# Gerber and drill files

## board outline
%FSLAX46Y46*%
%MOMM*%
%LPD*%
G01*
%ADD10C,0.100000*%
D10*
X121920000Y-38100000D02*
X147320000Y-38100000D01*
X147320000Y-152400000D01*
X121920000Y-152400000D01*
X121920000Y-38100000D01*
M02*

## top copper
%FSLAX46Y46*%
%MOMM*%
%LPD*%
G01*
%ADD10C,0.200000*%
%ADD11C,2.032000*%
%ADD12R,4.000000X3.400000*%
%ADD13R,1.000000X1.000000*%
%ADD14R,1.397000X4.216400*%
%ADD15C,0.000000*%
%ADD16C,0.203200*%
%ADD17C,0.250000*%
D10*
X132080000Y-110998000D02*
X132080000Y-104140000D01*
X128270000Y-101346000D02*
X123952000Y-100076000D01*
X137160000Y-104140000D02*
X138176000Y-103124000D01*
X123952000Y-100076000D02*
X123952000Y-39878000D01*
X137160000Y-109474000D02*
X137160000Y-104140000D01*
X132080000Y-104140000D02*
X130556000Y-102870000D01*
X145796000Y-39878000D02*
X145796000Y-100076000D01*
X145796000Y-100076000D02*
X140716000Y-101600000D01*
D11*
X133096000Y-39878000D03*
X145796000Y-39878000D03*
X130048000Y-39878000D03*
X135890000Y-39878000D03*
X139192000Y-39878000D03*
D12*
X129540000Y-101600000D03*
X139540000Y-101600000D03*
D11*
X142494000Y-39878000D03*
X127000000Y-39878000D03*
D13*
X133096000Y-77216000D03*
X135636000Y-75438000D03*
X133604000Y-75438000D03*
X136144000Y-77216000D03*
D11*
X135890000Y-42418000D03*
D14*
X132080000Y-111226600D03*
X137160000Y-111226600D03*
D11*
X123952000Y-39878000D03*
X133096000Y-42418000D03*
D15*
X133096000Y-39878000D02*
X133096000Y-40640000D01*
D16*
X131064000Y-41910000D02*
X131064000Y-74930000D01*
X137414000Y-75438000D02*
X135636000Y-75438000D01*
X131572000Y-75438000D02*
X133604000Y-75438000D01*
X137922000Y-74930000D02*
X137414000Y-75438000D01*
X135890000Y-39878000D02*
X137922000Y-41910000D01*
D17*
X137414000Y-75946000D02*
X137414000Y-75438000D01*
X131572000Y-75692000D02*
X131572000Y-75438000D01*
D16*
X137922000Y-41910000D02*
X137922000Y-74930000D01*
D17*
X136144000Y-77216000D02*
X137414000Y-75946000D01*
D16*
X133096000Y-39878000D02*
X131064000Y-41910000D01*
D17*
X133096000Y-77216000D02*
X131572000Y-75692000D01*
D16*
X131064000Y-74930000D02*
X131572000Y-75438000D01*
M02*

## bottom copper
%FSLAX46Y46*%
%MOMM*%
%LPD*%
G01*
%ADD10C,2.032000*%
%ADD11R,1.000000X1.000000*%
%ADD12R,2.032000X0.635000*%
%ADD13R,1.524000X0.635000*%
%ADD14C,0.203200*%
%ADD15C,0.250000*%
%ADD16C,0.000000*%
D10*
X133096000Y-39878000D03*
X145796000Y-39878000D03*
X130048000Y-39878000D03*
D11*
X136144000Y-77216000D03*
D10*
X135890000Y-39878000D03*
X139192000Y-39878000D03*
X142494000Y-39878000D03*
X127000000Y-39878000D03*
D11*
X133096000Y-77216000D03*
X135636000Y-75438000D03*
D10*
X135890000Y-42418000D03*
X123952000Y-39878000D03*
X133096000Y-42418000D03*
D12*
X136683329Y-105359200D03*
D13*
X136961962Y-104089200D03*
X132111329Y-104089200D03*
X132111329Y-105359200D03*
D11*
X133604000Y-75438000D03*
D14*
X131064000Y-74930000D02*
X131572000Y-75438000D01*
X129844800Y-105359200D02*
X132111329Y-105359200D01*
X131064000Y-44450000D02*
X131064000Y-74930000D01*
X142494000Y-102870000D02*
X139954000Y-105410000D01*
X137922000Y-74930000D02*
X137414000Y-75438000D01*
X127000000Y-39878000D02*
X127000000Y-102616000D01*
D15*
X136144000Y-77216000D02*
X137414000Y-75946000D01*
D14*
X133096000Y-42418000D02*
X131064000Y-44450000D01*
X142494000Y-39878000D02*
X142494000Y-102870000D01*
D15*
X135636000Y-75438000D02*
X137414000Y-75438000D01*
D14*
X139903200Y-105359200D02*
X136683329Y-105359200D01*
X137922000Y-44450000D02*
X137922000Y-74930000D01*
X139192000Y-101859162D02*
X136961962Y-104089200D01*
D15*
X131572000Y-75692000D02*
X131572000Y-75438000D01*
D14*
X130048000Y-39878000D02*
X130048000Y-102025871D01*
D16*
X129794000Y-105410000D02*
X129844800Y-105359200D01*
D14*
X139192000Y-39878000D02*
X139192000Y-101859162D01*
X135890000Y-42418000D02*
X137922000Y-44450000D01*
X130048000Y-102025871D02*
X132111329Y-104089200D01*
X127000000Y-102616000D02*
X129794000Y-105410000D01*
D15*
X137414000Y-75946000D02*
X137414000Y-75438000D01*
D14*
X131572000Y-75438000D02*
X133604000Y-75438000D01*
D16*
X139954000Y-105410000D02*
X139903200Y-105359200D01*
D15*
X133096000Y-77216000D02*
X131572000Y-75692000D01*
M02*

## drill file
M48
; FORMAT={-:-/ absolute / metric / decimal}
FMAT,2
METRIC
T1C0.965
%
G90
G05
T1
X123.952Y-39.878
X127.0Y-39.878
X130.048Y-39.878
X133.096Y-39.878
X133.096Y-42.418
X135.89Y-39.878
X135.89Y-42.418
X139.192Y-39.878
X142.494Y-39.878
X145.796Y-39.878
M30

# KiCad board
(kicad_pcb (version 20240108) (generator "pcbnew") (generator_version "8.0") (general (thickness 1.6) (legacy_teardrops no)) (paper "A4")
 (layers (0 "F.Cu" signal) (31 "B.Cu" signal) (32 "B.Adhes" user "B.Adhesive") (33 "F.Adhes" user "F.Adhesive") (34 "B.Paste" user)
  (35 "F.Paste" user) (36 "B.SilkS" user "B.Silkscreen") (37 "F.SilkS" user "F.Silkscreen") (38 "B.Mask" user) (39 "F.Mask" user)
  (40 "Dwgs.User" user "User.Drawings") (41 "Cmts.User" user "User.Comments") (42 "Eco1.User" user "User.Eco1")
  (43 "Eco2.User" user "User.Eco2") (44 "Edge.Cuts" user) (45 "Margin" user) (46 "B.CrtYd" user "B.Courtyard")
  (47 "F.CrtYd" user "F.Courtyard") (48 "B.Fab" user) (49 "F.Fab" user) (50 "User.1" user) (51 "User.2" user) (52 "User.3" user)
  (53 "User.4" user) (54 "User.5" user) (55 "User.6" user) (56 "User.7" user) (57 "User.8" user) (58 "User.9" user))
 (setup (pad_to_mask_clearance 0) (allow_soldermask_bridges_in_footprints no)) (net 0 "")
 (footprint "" (layer "F.Cu") (at 133.096 52.578)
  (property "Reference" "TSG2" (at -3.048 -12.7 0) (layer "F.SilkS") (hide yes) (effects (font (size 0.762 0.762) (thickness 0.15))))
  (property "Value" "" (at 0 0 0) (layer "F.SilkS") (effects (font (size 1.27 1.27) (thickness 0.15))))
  (pad "1" thru_hole circle (at 0 -12.7) (size 2.032 2.032) (drill 0.9652) (layers "*.Cu" "*.Mask") (remove_unused_layers no)))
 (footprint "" (layer "F.Cu") (at 145.796 39.878)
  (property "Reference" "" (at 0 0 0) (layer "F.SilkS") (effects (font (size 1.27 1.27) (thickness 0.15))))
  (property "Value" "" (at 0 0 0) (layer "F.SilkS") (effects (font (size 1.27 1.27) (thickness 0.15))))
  (pad "1" thru_hole circle (at 0 0) (size 2.032 2.032) (drill 0.9652) (layers "*.Cu" "*.Mask") (remove_unused_layers no)))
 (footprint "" (layer "F.Cu") (at 130.048 39.878)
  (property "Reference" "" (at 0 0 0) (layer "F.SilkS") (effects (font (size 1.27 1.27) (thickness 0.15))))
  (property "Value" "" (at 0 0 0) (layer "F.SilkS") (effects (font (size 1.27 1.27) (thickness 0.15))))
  (pad "1" thru_hole circle (at 0 0) (size 2.032 2.032) (drill 0.9652) (layers "*.Cu" "*.Mask") (remove_unused_layers no)))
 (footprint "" (layer "F.Cu") (at 136.144 77.216)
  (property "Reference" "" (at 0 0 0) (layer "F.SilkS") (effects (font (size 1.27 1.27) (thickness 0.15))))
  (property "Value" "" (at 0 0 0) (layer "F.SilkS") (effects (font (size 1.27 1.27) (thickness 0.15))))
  (pad "1" smd rect (at 0 0 180) (size 1 1) (layers "B.Cu" "B.Mask")))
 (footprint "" (layer "F.Cu") (at 135.89 52.578)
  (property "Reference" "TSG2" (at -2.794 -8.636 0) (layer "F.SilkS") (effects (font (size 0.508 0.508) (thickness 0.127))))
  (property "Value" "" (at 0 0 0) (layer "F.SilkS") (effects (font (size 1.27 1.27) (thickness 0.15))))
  (pad "1" thru_hole circle (at 0 -12.7) (size 2.032 2.032) (drill 0.9652) (layers "*.Cu" "*.Mask") (remove_unused_layers no)))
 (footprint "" (layer "F.Cu") (at 139.192 39.878)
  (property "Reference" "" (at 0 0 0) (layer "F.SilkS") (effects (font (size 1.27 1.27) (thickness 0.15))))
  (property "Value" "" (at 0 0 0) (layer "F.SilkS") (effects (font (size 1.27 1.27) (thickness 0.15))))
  (pad "1" thru_hole circle (at 0 0) (size 2.032 2.032) (drill 0.9652) (layers "*.Cu" "*.Mask") (remove_unused_layers no)))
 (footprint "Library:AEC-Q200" (layer "F.Cu") (at 134.62 107.95)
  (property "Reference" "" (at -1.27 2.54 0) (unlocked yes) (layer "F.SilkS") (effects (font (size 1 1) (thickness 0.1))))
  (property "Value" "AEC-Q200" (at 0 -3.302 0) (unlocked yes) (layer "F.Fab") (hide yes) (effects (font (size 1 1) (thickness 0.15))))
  (pad "1" smd rect (at -5.08 -6.35 180) (size 4 3.4) (layers "F.Cu" "F.Mask"))
  (pad "2" smd rect (at 4.92 -6.35 180) (size 4 3.4) (layers "F.Cu" "F.Mask")))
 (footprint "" (layer "F.Cu") (at 142.494 39.878)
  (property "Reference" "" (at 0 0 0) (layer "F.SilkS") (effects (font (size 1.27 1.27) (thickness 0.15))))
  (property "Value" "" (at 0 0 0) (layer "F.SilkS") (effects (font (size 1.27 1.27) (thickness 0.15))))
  (pad "1" thru_hole circle (at 0 0) (size 2.032 2.032) (drill 0.9652) (layers "*.Cu" "*.Mask") (remove_unused_layers no)))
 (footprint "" (layer "F.Cu") (at 127 39.878)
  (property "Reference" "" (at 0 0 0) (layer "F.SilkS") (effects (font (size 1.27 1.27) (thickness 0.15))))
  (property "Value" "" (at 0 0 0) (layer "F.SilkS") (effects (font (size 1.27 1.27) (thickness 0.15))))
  (pad "1" thru_hole circle (at 0 0) (size 2.032 2.032) (drill 0.9652) (layers "*.Cu" "*.Mask") (remove_unused_layers no)))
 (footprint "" (layer "F.Cu") (at 133.096 77.216)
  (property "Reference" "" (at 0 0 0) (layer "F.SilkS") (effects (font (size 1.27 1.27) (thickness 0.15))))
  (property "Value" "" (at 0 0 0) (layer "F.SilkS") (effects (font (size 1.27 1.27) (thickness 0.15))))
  (pad "1" smd rect (at 0 0) (size 1 1) (layers "F.Cu" "F.Mask")))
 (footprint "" (layer "F.Cu") (at 133.096 77.216)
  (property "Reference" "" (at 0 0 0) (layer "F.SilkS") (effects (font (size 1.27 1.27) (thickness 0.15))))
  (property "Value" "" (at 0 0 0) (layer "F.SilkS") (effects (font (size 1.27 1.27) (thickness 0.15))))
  (pad "1" smd rect (at 0 0 180) (size 1 1) (layers "B.Cu" "B.Mask")))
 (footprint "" (layer "F.Cu") (at 135.636 75.438)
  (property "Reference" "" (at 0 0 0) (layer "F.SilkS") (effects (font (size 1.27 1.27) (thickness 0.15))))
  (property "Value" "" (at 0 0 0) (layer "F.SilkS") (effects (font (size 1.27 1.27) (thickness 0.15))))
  (pad "1" smd rect (at 0 0) (size 1 1) (layers "F.Cu" "F.Mask")))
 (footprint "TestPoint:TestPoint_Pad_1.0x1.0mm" (layer "F.Cu") (at 133.604 75.438)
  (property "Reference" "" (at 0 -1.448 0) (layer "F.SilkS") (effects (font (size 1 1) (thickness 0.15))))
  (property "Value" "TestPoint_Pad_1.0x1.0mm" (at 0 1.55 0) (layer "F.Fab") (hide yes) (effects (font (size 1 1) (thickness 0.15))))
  (pad "1" smd rect (at 0 0) (size 1 1) (layers "F.Cu" "F.Mask")))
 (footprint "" (layer "F.Cu") (at 136.144 77.216)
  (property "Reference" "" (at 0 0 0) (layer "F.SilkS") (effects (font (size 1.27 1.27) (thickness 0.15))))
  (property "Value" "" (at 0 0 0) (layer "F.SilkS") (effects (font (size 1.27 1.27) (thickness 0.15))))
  (pad "1" smd rect (at 0 0) (size 1 1) (layers "F.Cu" "F.Mask")))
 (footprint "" (layer "F.Cu") (at 135.636 75.438)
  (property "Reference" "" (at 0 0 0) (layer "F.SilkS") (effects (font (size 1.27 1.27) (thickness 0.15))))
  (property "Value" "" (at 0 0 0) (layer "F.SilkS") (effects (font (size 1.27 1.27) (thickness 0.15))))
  (pad "1" smd rect (at 0 0 180) (size 1 1) (layers "B.Cu" "B.Mask")))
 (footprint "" (layer "F.Cu") (at 135.89 55.118)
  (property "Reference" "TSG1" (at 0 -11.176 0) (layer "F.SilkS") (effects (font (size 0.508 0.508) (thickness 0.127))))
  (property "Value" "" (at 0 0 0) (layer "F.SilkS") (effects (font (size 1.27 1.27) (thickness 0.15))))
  (pad "1" thru_hole circle (at 0 -12.7) (size 2.032 2.032) (drill 0.9652) (layers "*.Cu" "*.Mask") (remove_unused_layers no)))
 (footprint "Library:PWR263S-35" (layer "F.Cu") (at 135.89 112.268)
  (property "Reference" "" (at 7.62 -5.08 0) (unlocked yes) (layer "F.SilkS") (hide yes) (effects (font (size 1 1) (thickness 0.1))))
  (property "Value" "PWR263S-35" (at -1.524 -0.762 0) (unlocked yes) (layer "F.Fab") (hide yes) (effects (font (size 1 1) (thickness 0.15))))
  (pad "1" smd rect (at -3.81 -1.0414) (size 1.397 4.2164) (layers "F.Cu" "F.Mask"))
  (pad "2" smd rect (at 1.27 -1.0414) (size 1.397 4.2164) (layers "F.Cu" "F.Mask")))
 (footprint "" (layer "F.Cu") (at 123.952 39.878)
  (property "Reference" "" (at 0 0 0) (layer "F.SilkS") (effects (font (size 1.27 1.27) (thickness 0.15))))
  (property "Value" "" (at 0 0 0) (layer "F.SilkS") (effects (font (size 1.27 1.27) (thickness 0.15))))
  (pad "1" thru_hole circle (at 0 0) (size 2.032 2.032) (drill 0.9652) (layers "*.Cu" "*.Mask") (remove_unused_layers no)))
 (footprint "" (layer "F.Cu") (at 133.096 55.118)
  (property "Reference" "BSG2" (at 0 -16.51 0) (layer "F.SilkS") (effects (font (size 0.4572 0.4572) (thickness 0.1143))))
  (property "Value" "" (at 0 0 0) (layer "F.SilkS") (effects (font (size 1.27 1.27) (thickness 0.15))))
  (pad "1" thru_hole circle (at 0 -12.7) (size 2.032 2.032) (drill 0.9652) (layers "*.Cu" "*.Mask") (remove_unused_layers no)))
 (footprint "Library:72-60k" (layer "B.Cu") (at 132.873329 109.1692 180)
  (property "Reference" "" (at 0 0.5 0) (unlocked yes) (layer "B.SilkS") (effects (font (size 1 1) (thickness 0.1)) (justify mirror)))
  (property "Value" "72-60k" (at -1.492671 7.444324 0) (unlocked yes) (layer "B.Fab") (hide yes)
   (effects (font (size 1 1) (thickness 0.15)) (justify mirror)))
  (pad "1" smd rect (at -3.81 3.81) (size 2.032 0.635) (layers "B.Cu" "B.Mask"))
  (pad "2" smd rect (at -4.088633 5.08) (size 1.524 0.635) (layers "B.Cu" "B.Mask"))
  (pad "3" smd rect (at 0.762 5.08) (size 1.524 0.635) (layers "B.Cu" "B.Mask"))
  (pad "4" smd rect (at 0.762 3.81) (size 1.524 0.635) (layers "B.Cu" "B.Mask")))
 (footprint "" (layer "B.Cu") (at 133.604 75.438 180)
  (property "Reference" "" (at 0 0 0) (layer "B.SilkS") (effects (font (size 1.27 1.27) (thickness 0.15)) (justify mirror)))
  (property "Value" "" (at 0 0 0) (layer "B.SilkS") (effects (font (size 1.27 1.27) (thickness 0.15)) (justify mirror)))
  (pad "1" smd rect (at 0 0 180) (size 1 1) (layers "B.Cu" "B.Mask")))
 (gr_line (start 132.08 110.998) (end 132.08 104.14) (stroke (width 0.2) (type default)) (layer "F.Cu"))
 (gr_line (start 128.27 101.346) (end 123.952 100.076) (stroke (width 0.2) (type default)) (layer "F.Cu"))
 (gr_line (start 137.16 104.14) (end 138.176 103.124) (stroke (width 0.2) (type default)) (layer "F.Cu"))
 (gr_line (start 123.952 100.076) (end 123.952 39.878) (stroke (width 0.2) (type default)) (layer "F.Cu"))
 (gr_line (start 137.16 109.474) (end 137.16 104.14) (stroke (width 0.2) (type default)) (layer "F.Cu"))
 (gr_line (start 132.08 104.14) (end 130.556 102.87) (stroke (width 0.2) (type default)) (layer "F.Cu"))
 (gr_line (start 145.796 39.878) (end 145.796 100.076) (stroke (width 0.2) (type default)) (layer "F.Cu"))
 (gr_line (start 145.796 100.076) (end 140.716 101.6) (stroke (width 0.2) (type default)) (layer "F.Cu"))
 (gr_rect (start 121.92 38.1) (end 147.32 152.4) (stroke (width 0.1) (type default)) (fill none) (layer "Edge.Cuts"))
 (segment (start 133.096 39.878) (end 133.096 40.64) (width 0) (layer "F.Cu") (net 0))
 (segment (start 131.064 41.91) (end 131.064 74.93) (width 0.2032) (layer "F.Cu") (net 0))
 (segment (start 137.414 75.438) (end 135.636 75.438) (width 0.2032) (layer "F.Cu") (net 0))
 (segment (start 131.572 75.438) (end 133.604 75.438) (width 0.2032) (layer "F.Cu") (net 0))
 (segment (start 137.922 74.93) (end 137.414 75.438) (width 0.2032) (layer "F.Cu") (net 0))
 (segment (start 135.89 39.878) (end 137.922 41.91) (width 0.2032) (layer "F.Cu") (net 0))
 (segment (start 137.414 75.946) (end 137.414 75.438) (width 0.25) (layer "F.Cu") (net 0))
 (segment (start 131.572 75.692) (end 131.572 75.438) (width 0.25) (layer "F.Cu") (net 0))
 (segment (start 137.922 41.91) (end 137.922 74.93) (width 0.2032) (layer "F.Cu") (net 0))
 (segment (start 136.144 77.216) (end 137.414 75.946) (width 0.25) (layer "F.Cu") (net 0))
 (segment (start 133.096 39.878) (end 131.064 41.91) (width 0.2032) (layer "F.Cu") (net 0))
 (segment (start 133.096 77.216) (end 131.572 75.692) (width 0.25) (layer "F.Cu") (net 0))
 (segment (start 131.064 74.93) (end 131.572 75.438) (width 0.2032) (layer "F.Cu") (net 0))
 (segment (start 131.064 74.93) (end 131.572 75.438) (width 0.2032) (layer "B.Cu") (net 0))
 (segment (start 129.8448 105.3592) (end 132.111329 105.3592) (width 0.2032) (layer "B.Cu") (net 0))
 (segment (start 131.064 44.45) (end 131.064 74.93) (width 0.2032) (layer "B.Cu") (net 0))
 (segment (start 142.494 102.87) (end 139.954 105.41) (width 0.2032) (layer "B.Cu") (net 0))
 (segment (start 137.922 74.93) (end 137.414 75.438) (width 0.2032) (layer "B.Cu") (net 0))
 (segment (start 127 39.878) (end 127 102.616) (width 0.2032) (layer "B.Cu") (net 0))
 (segment (start 136.144 77.216) (end 137.414 75.946) (width 0.25) (layer "B.Cu") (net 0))
 (segment (start 133.096 42.418) (end 131.064 44.45) (width 0.2032) (layer "B.Cu") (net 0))
 (segment (start 142.494 39.878) (end 142.494 102.87) (width 0.2032) (layer "B.Cu") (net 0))
 (segment (start 135.636 75.438) (end 137.414 75.438) (width 0.25) (layer "B.Cu") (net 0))
 (segment (start 139.9032 105.3592) (end 136.683329 105.3592) (width 0.2032) (layer "B.Cu") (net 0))
 (segment (start 137.922 44.45) (end 137.922 74.93) (width 0.2032) (layer "B.Cu") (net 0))
 (segment (start 139.192 101.859162) (end 136.961962 104.0892) (width 0.2032) (layer "B.Cu") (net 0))
 (segment (start 131.572 75.692) (end 131.572 75.438) (width 0.25) (layer "B.Cu") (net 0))
 (segment (start 130.048 39.878) (end 130.048 102.025871) (width 0.2032) (layer "B.Cu") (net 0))
 (segment (start 129.794 105.41) (end 129.8448 105.3592) (width 0) (layer "B.Cu") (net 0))
 (segment (start 139.192 39.878) (end 139.192 101.859162) (width 0.2032) (layer "B.Cu") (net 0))
 (segment (start 135.89 42.418) (end 137.922 44.45) (width 0.2032) (layer "B.Cu") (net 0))
 (segment (start 130.048 102.025871) (end 132.111329 104.0892) (width 0.2032) (layer "B.Cu") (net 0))
 (segment (start 127 102.616) (end 129.794 105.41) (width 0.2032) (layer "B.Cu") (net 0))
 (segment (start 137.414 75.946) (end 137.414 75.438) (width 0.25) (layer "B.Cu") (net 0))
 (segment (start 131.572 75.438) (end 133.604 75.438) (width 0.2032) (layer "B.Cu") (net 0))
 (segment (start 139.954 105.41) (end 139.9032 105.3592) (width 0) (layer "B.Cu") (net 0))
 (segment (start 133.096 77.216) (end 131.572 75.692) (width 0.25) (layer "B.Cu") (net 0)))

